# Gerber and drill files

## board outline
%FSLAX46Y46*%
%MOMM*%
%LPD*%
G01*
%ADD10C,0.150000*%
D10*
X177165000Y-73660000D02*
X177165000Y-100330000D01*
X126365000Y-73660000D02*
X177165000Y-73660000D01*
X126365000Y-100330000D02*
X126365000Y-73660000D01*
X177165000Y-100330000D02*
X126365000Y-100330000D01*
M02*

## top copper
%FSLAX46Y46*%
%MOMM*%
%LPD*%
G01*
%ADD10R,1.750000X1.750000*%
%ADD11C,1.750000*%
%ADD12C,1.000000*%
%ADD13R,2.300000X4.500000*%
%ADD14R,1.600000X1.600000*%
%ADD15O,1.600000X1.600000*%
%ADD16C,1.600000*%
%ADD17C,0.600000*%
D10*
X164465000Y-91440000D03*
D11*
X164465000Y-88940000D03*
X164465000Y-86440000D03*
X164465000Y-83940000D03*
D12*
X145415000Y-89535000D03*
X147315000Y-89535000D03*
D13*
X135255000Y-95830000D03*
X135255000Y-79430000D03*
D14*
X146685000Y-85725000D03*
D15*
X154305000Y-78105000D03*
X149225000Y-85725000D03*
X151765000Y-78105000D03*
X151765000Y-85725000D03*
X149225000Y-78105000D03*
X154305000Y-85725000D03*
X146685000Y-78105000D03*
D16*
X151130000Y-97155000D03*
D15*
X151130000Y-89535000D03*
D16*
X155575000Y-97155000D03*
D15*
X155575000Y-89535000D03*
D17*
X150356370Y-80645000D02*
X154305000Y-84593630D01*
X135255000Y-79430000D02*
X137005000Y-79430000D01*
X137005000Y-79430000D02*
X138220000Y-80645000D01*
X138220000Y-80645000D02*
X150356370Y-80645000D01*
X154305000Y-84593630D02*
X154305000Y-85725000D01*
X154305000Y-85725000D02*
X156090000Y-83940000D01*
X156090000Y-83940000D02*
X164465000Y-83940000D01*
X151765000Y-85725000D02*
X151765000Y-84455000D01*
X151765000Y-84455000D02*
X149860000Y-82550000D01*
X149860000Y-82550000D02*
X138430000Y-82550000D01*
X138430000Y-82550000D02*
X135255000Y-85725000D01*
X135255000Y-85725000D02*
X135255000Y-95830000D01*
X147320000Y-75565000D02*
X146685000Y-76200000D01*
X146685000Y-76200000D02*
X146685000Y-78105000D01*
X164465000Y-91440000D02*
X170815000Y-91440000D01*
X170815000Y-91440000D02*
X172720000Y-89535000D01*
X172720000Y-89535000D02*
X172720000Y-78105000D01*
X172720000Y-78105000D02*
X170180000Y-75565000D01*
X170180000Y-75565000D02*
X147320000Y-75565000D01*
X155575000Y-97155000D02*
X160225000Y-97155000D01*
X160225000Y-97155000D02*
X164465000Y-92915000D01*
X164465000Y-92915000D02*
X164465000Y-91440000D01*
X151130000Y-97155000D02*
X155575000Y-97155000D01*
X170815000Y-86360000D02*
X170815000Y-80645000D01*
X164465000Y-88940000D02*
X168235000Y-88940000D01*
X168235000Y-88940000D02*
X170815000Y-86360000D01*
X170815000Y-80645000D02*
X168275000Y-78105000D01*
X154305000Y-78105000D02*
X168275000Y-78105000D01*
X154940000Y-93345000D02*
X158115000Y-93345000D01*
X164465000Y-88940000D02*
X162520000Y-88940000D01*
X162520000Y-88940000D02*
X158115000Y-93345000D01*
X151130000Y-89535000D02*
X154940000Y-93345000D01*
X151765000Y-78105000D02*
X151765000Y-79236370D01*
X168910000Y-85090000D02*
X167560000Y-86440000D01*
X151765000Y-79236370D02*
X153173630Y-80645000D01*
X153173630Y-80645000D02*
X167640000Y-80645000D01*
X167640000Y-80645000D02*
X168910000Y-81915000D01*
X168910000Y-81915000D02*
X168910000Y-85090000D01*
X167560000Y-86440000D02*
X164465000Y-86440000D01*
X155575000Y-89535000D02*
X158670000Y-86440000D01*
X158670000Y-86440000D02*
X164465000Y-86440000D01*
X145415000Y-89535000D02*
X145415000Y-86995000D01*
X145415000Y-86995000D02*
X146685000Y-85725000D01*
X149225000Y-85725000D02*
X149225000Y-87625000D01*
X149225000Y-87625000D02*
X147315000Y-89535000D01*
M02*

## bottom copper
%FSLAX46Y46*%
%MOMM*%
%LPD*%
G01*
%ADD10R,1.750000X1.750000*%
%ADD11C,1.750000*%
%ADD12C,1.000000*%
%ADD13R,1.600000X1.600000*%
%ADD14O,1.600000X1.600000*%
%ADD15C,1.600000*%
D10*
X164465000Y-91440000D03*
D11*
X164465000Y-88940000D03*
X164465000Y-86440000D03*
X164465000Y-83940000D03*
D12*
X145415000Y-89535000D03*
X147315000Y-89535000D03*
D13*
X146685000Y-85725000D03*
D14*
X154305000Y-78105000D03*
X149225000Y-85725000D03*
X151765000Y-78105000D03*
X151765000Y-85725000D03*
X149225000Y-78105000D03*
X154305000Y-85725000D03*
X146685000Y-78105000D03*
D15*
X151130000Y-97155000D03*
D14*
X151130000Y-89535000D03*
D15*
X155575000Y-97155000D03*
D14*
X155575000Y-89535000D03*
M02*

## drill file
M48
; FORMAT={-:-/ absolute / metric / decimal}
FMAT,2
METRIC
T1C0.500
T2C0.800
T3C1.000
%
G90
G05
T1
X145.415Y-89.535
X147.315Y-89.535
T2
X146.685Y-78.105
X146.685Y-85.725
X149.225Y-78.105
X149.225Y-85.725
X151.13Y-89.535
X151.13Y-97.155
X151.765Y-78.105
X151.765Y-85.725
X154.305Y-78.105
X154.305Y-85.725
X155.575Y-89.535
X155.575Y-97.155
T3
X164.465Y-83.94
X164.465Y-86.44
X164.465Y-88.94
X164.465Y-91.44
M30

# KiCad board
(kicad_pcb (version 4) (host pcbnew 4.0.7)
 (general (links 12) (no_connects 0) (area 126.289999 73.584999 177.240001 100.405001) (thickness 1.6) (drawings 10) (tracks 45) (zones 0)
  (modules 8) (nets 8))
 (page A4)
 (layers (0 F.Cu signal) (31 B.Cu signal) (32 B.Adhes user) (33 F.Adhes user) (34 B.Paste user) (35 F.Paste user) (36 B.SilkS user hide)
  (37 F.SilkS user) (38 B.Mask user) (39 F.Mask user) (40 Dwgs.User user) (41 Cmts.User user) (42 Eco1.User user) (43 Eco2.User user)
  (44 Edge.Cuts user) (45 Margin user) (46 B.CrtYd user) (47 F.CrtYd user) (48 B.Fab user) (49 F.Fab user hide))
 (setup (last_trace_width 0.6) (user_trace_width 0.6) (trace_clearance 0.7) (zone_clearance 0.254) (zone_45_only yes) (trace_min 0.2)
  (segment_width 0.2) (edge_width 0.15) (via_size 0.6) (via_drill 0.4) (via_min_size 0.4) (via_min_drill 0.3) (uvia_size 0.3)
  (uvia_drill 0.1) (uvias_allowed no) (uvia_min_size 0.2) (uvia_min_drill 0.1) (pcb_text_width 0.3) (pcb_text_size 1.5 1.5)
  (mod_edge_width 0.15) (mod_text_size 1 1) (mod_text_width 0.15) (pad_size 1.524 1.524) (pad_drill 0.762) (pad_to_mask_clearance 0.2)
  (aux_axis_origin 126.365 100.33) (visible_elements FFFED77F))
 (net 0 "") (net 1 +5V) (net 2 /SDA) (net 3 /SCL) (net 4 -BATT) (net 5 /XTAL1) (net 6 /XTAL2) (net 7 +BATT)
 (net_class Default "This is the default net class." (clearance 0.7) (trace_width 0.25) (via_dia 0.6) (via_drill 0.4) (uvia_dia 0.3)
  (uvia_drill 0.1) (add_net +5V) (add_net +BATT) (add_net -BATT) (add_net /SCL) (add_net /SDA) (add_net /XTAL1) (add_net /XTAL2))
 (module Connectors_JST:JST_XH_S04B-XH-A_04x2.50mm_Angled (layer F.Cu) (at 164.465 91.44 90)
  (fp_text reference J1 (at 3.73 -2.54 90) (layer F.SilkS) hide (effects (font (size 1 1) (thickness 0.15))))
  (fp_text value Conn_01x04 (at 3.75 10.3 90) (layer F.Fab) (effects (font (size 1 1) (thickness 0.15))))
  (pad 1 thru_hole rect (at 0 0 90) (size 1.75 1.75) (drill 1) (layers *.Cu *.Mask F.SilkS) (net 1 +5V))
  (pad 2 thru_hole circle (at 2.5 0 90) (size 1.75 1.75) (drill 1) (layers *.Cu *.Mask F.SilkS) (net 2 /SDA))
  (pad 3 thru_hole circle (at 5 0 90) (size 1.75 1.75) (drill 1) (layers *.Cu *.Mask F.SilkS) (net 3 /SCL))
  (pad 4 thru_hole circle (at 7.5 0 90) (size 1.75 1.75) (drill 1) (layers *.Cu *.Mask F.SilkS) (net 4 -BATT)))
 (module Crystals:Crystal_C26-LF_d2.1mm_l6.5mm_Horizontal (layer F.Cu) (at 145.415 89.535)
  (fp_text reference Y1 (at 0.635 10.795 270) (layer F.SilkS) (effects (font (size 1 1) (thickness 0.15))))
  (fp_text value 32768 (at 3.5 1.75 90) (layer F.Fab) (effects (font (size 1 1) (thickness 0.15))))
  (pad 1 thru_hole circle (at 0 0) (size 1 1) (drill 0.5) (layers *.Cu *.Mask) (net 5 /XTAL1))
  (pad 2 thru_hole circle (at 1.9 0) (size 1 1) (drill 0.5) (layers *.Cu *.Mask) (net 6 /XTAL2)))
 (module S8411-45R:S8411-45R (layer F.Cu) (at 135.255 87.63)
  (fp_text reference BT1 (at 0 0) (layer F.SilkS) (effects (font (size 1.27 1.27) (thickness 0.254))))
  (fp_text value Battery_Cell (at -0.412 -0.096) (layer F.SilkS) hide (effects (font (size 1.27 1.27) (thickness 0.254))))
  (pad 1 smd rect (at 0 8.2) (size 2.3 4.5) (layers F.Cu F.Paste F.Mask) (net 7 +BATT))
  (pad 2 smd rect (at 0 -8.2) (size 2.3 4.5) (layers F.Cu F.Paste F.Mask) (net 4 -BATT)))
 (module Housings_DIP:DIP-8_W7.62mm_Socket (layer F.Cu) (at 146.685 85.725 90)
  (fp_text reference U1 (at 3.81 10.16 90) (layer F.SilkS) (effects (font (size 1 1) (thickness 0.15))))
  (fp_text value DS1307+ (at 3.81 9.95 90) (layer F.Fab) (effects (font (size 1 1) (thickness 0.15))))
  (pad 1 thru_hole rect (at 0 0 90) (size 1.6 1.6) (drill 0.8) (layers *.Cu *.Mask) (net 5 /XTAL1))
  (pad 5 thru_hole oval (at 7.62 7.62 90) (size 1.6 1.6) (drill 0.8) (layers *.Cu *.Mask) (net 2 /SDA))
  (pad 2 thru_hole oval (at 0 2.54 90) (size 1.6 1.6) (drill 0.8) (layers *.Cu *.Mask) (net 6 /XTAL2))
  (pad 6 thru_hole oval (at 7.62 5.08 90) (size 1.6 1.6) (drill 0.8) (layers *.Cu *.Mask) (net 3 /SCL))
  (pad 3 thru_hole oval (at 0 5.08 90) (size 1.6 1.6) (drill 0.8) (layers *.Cu *.Mask) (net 7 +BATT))
  (pad 7 thru_hole oval (at 7.62 2.54 90) (size 1.6 1.6) (drill 0.8) (layers *.Cu *.Mask))
  (pad 4 thru_hole oval (at 0 7.62 90) (size 1.6 1.6) (drill 0.8) (layers *.Cu *.Mask) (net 4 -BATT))
  (pad 8 thru_hole oval (at 7.62 0 90) (size 1.6 1.6) (drill 0.8) (layers *.Cu *.Mask) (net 1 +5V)))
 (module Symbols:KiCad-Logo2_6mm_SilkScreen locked (layer B.Cu) (at 142.24 91.44 270)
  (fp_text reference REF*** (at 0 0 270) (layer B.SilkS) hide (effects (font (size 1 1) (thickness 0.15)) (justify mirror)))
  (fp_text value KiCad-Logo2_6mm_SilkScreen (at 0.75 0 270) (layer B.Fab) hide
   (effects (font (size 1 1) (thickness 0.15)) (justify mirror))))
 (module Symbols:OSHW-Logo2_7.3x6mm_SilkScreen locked (layer B.Cu) (at 142.24 80.645 270)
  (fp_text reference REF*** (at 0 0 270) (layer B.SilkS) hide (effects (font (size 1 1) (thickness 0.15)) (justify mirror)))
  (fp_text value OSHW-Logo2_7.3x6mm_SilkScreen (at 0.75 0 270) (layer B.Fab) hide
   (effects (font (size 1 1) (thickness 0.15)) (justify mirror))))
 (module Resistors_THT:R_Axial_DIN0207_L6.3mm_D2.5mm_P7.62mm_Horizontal (layer F.Cu) (at 151.13 97.155 90)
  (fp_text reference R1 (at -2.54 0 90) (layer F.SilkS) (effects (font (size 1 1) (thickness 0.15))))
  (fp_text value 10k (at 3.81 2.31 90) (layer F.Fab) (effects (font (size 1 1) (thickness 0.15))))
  (pad 1 thru_hole circle (at 0 0 90) (size 1.6 1.6) (drill 0.8) (layers *.Cu *.Mask) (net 1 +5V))
  (pad 2 thru_hole oval (at 7.62 0 90) (size 1.6 1.6) (drill 0.8) (layers *.Cu *.Mask) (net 2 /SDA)))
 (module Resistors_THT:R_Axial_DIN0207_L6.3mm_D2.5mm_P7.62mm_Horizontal (layer F.Cu) (at 155.575 97.155 90)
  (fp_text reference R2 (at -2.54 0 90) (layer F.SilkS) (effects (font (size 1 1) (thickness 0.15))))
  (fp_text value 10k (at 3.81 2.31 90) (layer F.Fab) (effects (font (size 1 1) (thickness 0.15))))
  (pad 1 thru_hole circle (at 0 0 90) (size 1.6 1.6) (drill 0.8) (layers *.Cu *.Mask) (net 1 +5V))
  (pad 2 thru_hole oval (at 7.62 0 90) (size 1.6 1.6) (drill 0.8) (layers *.Cu *.Mask) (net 3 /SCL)))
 (gr_line (start 177.165 73.66) (end 177.165 100.33) (layer Edge.Cuts) (width 0.15))
 (gr_line (start 126.365 73.66) (end 177.165 73.66) (layer Edge.Cuts) (width 0.15))
 (gr_line (start 126.365 100.33) (end 126.365 73.66) (layer Edge.Cuts) (width 0.15))
 (gr_line (start 177.165 100.33) (end 126.365 100.33) (layer Edge.Cuts) (width 0.15))
 (segment (start 150.35637 80.645) (end 154.305 84.59363) (width 0.6) (layer F.Cu) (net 4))
 (segment (start 135.255 79.43) (end 137.005 79.43) (width 0.6) (layer F.Cu) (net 4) (status 10))
 (segment (start 137.005 79.43) (end 138.22 80.645) (width 0.6) (layer F.Cu) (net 4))
 (segment (start 138.22 80.645) (end 150.35637 80.645) (width 0.6) (layer F.Cu) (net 4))
 (segment (start 154.305 84.59363) (end 154.305 85.725) (width 0.6) (layer F.Cu) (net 4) (status 20))
 (segment (start 154.305 85.725) (end 156.09 83.94) (width 0.6) (layer F.Cu) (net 4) (status 10))
 (segment (start 156.09 83.94) (end 164.465 83.94) (width 0.6) (layer F.Cu) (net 4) (status 20))
 (segment (start 151.765 85.725) (end 151.765 84.455) (width 0.6) (layer F.Cu) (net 7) (status 10))
 (segment (start 151.765 84.455) (end 149.86 82.55) (width 0.6) (layer F.Cu) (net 7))
 (segment (start 149.86 82.55) (end 138.43 82.55) (width 0.6) (layer F.Cu) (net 7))
 (segment (start 138.43 82.55) (end 135.255 85.725) (width 0.6) (layer F.Cu) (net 7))
 (segment (start 135.255 85.725) (end 135.255 95.83) (width 0.6) (layer F.Cu) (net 7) (status 20))
 (segment (start 147.32 75.565) (end 146.685 76.2) (width 0.6) (layer F.Cu) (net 1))
 (segment (start 146.685 76.2) (end 146.685 78.105) (width 0.6) (layer F.Cu) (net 1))
 (segment (start 164.465 91.44) (end 170.815 91.44) (width 0.6) (layer F.Cu) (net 1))
 (segment (start 170.815 91.44) (end 172.72 89.535) (width 0.6) (layer F.Cu) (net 1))
 (segment (start 172.72 89.535) (end 172.72 78.105) (width 0.6) (layer F.Cu) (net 1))
 (segment (start 172.72 78.105) (end 170.18 75.565) (width 0.6) (layer F.Cu) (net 1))
 (segment (start 170.18 75.565) (end 147.32 75.565) (width 0.6) (layer F.Cu) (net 1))
 (segment (start 155.575 97.155) (end 160.225 97.155) (width 0.6) (layer F.Cu) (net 1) (status 10))
 (segment (start 160.225 97.155) (end 164.465 92.915) (width 0.6) (layer F.Cu) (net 1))
 (segment (start 164.465 92.915) (end 164.465 91.44) (width 0.6) (layer F.Cu) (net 1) (status 20))
 (segment (start 151.13 97.155) (end 155.575 97.155) (width 0.6) (layer F.Cu) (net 1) (status 30))
 (segment (start 170.815 86.36) (end 170.815 80.645) (width 0.6) (layer F.Cu) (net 2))
 (segment (start 164.465 88.94) (end 168.235 88.94) (width 0.6) (layer F.Cu) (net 2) (status 10))
 (segment (start 168.235 88.94) (end 170.815 86.36) (width 0.6) (layer F.Cu) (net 2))
 (segment (start 170.815 80.645) (end 168.275 78.105) (width 0.6) (layer F.Cu) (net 2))
 (segment (start 154.305 78.105) (end 168.275 78.105) (width 0.6) (layer F.Cu) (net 2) (status 10))
 (segment (start 154.94 93.345) (end 158.115 93.345) (width 0.6) (layer F.Cu) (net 2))
 (segment (start 164.465 88.94) (end 162.52 88.94) (width 0.6) (layer F.Cu) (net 2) (status 10))
 (segment (start 162.52 88.94) (end 158.115 93.345) (width 0.6) (layer F.Cu) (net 2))
 (segment (start 151.13 89.535) (end 154.94 93.345) (width 0.6) (layer F.Cu) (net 2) (status 10))
 (segment (start 151.765 78.105) (end 151.765 79.23637) (width 0.6) (layer F.Cu) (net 3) (status 10))
 (segment (start 168.91 85.09) (end 167.56 86.44) (width 0.6) (layer F.Cu) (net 3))
 (segment (start 151.765 79.23637) (end 153.17363 80.645) (width 0.6) (layer F.Cu) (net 3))
 (segment (start 153.17363 80.645) (end 167.64 80.645) (width 0.6) (layer F.Cu) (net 3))
 (segment (start 167.64 80.645) (end 168.91 81.915) (width 0.6) (layer F.Cu) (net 3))
 (segment (start 168.91 81.915) (end 168.91 85.09) (width 0.6) (layer F.Cu) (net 3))
 (segment (start 167.56 86.44) (end 164.465 86.44) (width 0.6) (layer F.Cu) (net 3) (status 20))
 (segment (start 155.575 89.535) (end 158.67 86.44) (width 0.6) (layer F.Cu) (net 3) (status 10))
 (segment (start 158.67 86.44) (end 164.465 86.44) (width 0.6) (layer F.Cu) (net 3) (status 20))
 (segment (start 145.415 89.535) (end 145.415 86.995) (width 0.6) (layer F.Cu) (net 5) (status 10))
 (segment (start 145.415 86.995) (end 146.685 85.725) (width 0.6) (layer F.Cu) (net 5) (status 20))
 (segment (start 149.225 85.725) (end 149.225 87.625) (width 0.6) (layer F.Cu) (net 6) (status 10))
 (segment (start 149.225 87.625) (end 147.315 89.535) (width 0.6) (layer F.Cu) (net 6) (status 20)))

